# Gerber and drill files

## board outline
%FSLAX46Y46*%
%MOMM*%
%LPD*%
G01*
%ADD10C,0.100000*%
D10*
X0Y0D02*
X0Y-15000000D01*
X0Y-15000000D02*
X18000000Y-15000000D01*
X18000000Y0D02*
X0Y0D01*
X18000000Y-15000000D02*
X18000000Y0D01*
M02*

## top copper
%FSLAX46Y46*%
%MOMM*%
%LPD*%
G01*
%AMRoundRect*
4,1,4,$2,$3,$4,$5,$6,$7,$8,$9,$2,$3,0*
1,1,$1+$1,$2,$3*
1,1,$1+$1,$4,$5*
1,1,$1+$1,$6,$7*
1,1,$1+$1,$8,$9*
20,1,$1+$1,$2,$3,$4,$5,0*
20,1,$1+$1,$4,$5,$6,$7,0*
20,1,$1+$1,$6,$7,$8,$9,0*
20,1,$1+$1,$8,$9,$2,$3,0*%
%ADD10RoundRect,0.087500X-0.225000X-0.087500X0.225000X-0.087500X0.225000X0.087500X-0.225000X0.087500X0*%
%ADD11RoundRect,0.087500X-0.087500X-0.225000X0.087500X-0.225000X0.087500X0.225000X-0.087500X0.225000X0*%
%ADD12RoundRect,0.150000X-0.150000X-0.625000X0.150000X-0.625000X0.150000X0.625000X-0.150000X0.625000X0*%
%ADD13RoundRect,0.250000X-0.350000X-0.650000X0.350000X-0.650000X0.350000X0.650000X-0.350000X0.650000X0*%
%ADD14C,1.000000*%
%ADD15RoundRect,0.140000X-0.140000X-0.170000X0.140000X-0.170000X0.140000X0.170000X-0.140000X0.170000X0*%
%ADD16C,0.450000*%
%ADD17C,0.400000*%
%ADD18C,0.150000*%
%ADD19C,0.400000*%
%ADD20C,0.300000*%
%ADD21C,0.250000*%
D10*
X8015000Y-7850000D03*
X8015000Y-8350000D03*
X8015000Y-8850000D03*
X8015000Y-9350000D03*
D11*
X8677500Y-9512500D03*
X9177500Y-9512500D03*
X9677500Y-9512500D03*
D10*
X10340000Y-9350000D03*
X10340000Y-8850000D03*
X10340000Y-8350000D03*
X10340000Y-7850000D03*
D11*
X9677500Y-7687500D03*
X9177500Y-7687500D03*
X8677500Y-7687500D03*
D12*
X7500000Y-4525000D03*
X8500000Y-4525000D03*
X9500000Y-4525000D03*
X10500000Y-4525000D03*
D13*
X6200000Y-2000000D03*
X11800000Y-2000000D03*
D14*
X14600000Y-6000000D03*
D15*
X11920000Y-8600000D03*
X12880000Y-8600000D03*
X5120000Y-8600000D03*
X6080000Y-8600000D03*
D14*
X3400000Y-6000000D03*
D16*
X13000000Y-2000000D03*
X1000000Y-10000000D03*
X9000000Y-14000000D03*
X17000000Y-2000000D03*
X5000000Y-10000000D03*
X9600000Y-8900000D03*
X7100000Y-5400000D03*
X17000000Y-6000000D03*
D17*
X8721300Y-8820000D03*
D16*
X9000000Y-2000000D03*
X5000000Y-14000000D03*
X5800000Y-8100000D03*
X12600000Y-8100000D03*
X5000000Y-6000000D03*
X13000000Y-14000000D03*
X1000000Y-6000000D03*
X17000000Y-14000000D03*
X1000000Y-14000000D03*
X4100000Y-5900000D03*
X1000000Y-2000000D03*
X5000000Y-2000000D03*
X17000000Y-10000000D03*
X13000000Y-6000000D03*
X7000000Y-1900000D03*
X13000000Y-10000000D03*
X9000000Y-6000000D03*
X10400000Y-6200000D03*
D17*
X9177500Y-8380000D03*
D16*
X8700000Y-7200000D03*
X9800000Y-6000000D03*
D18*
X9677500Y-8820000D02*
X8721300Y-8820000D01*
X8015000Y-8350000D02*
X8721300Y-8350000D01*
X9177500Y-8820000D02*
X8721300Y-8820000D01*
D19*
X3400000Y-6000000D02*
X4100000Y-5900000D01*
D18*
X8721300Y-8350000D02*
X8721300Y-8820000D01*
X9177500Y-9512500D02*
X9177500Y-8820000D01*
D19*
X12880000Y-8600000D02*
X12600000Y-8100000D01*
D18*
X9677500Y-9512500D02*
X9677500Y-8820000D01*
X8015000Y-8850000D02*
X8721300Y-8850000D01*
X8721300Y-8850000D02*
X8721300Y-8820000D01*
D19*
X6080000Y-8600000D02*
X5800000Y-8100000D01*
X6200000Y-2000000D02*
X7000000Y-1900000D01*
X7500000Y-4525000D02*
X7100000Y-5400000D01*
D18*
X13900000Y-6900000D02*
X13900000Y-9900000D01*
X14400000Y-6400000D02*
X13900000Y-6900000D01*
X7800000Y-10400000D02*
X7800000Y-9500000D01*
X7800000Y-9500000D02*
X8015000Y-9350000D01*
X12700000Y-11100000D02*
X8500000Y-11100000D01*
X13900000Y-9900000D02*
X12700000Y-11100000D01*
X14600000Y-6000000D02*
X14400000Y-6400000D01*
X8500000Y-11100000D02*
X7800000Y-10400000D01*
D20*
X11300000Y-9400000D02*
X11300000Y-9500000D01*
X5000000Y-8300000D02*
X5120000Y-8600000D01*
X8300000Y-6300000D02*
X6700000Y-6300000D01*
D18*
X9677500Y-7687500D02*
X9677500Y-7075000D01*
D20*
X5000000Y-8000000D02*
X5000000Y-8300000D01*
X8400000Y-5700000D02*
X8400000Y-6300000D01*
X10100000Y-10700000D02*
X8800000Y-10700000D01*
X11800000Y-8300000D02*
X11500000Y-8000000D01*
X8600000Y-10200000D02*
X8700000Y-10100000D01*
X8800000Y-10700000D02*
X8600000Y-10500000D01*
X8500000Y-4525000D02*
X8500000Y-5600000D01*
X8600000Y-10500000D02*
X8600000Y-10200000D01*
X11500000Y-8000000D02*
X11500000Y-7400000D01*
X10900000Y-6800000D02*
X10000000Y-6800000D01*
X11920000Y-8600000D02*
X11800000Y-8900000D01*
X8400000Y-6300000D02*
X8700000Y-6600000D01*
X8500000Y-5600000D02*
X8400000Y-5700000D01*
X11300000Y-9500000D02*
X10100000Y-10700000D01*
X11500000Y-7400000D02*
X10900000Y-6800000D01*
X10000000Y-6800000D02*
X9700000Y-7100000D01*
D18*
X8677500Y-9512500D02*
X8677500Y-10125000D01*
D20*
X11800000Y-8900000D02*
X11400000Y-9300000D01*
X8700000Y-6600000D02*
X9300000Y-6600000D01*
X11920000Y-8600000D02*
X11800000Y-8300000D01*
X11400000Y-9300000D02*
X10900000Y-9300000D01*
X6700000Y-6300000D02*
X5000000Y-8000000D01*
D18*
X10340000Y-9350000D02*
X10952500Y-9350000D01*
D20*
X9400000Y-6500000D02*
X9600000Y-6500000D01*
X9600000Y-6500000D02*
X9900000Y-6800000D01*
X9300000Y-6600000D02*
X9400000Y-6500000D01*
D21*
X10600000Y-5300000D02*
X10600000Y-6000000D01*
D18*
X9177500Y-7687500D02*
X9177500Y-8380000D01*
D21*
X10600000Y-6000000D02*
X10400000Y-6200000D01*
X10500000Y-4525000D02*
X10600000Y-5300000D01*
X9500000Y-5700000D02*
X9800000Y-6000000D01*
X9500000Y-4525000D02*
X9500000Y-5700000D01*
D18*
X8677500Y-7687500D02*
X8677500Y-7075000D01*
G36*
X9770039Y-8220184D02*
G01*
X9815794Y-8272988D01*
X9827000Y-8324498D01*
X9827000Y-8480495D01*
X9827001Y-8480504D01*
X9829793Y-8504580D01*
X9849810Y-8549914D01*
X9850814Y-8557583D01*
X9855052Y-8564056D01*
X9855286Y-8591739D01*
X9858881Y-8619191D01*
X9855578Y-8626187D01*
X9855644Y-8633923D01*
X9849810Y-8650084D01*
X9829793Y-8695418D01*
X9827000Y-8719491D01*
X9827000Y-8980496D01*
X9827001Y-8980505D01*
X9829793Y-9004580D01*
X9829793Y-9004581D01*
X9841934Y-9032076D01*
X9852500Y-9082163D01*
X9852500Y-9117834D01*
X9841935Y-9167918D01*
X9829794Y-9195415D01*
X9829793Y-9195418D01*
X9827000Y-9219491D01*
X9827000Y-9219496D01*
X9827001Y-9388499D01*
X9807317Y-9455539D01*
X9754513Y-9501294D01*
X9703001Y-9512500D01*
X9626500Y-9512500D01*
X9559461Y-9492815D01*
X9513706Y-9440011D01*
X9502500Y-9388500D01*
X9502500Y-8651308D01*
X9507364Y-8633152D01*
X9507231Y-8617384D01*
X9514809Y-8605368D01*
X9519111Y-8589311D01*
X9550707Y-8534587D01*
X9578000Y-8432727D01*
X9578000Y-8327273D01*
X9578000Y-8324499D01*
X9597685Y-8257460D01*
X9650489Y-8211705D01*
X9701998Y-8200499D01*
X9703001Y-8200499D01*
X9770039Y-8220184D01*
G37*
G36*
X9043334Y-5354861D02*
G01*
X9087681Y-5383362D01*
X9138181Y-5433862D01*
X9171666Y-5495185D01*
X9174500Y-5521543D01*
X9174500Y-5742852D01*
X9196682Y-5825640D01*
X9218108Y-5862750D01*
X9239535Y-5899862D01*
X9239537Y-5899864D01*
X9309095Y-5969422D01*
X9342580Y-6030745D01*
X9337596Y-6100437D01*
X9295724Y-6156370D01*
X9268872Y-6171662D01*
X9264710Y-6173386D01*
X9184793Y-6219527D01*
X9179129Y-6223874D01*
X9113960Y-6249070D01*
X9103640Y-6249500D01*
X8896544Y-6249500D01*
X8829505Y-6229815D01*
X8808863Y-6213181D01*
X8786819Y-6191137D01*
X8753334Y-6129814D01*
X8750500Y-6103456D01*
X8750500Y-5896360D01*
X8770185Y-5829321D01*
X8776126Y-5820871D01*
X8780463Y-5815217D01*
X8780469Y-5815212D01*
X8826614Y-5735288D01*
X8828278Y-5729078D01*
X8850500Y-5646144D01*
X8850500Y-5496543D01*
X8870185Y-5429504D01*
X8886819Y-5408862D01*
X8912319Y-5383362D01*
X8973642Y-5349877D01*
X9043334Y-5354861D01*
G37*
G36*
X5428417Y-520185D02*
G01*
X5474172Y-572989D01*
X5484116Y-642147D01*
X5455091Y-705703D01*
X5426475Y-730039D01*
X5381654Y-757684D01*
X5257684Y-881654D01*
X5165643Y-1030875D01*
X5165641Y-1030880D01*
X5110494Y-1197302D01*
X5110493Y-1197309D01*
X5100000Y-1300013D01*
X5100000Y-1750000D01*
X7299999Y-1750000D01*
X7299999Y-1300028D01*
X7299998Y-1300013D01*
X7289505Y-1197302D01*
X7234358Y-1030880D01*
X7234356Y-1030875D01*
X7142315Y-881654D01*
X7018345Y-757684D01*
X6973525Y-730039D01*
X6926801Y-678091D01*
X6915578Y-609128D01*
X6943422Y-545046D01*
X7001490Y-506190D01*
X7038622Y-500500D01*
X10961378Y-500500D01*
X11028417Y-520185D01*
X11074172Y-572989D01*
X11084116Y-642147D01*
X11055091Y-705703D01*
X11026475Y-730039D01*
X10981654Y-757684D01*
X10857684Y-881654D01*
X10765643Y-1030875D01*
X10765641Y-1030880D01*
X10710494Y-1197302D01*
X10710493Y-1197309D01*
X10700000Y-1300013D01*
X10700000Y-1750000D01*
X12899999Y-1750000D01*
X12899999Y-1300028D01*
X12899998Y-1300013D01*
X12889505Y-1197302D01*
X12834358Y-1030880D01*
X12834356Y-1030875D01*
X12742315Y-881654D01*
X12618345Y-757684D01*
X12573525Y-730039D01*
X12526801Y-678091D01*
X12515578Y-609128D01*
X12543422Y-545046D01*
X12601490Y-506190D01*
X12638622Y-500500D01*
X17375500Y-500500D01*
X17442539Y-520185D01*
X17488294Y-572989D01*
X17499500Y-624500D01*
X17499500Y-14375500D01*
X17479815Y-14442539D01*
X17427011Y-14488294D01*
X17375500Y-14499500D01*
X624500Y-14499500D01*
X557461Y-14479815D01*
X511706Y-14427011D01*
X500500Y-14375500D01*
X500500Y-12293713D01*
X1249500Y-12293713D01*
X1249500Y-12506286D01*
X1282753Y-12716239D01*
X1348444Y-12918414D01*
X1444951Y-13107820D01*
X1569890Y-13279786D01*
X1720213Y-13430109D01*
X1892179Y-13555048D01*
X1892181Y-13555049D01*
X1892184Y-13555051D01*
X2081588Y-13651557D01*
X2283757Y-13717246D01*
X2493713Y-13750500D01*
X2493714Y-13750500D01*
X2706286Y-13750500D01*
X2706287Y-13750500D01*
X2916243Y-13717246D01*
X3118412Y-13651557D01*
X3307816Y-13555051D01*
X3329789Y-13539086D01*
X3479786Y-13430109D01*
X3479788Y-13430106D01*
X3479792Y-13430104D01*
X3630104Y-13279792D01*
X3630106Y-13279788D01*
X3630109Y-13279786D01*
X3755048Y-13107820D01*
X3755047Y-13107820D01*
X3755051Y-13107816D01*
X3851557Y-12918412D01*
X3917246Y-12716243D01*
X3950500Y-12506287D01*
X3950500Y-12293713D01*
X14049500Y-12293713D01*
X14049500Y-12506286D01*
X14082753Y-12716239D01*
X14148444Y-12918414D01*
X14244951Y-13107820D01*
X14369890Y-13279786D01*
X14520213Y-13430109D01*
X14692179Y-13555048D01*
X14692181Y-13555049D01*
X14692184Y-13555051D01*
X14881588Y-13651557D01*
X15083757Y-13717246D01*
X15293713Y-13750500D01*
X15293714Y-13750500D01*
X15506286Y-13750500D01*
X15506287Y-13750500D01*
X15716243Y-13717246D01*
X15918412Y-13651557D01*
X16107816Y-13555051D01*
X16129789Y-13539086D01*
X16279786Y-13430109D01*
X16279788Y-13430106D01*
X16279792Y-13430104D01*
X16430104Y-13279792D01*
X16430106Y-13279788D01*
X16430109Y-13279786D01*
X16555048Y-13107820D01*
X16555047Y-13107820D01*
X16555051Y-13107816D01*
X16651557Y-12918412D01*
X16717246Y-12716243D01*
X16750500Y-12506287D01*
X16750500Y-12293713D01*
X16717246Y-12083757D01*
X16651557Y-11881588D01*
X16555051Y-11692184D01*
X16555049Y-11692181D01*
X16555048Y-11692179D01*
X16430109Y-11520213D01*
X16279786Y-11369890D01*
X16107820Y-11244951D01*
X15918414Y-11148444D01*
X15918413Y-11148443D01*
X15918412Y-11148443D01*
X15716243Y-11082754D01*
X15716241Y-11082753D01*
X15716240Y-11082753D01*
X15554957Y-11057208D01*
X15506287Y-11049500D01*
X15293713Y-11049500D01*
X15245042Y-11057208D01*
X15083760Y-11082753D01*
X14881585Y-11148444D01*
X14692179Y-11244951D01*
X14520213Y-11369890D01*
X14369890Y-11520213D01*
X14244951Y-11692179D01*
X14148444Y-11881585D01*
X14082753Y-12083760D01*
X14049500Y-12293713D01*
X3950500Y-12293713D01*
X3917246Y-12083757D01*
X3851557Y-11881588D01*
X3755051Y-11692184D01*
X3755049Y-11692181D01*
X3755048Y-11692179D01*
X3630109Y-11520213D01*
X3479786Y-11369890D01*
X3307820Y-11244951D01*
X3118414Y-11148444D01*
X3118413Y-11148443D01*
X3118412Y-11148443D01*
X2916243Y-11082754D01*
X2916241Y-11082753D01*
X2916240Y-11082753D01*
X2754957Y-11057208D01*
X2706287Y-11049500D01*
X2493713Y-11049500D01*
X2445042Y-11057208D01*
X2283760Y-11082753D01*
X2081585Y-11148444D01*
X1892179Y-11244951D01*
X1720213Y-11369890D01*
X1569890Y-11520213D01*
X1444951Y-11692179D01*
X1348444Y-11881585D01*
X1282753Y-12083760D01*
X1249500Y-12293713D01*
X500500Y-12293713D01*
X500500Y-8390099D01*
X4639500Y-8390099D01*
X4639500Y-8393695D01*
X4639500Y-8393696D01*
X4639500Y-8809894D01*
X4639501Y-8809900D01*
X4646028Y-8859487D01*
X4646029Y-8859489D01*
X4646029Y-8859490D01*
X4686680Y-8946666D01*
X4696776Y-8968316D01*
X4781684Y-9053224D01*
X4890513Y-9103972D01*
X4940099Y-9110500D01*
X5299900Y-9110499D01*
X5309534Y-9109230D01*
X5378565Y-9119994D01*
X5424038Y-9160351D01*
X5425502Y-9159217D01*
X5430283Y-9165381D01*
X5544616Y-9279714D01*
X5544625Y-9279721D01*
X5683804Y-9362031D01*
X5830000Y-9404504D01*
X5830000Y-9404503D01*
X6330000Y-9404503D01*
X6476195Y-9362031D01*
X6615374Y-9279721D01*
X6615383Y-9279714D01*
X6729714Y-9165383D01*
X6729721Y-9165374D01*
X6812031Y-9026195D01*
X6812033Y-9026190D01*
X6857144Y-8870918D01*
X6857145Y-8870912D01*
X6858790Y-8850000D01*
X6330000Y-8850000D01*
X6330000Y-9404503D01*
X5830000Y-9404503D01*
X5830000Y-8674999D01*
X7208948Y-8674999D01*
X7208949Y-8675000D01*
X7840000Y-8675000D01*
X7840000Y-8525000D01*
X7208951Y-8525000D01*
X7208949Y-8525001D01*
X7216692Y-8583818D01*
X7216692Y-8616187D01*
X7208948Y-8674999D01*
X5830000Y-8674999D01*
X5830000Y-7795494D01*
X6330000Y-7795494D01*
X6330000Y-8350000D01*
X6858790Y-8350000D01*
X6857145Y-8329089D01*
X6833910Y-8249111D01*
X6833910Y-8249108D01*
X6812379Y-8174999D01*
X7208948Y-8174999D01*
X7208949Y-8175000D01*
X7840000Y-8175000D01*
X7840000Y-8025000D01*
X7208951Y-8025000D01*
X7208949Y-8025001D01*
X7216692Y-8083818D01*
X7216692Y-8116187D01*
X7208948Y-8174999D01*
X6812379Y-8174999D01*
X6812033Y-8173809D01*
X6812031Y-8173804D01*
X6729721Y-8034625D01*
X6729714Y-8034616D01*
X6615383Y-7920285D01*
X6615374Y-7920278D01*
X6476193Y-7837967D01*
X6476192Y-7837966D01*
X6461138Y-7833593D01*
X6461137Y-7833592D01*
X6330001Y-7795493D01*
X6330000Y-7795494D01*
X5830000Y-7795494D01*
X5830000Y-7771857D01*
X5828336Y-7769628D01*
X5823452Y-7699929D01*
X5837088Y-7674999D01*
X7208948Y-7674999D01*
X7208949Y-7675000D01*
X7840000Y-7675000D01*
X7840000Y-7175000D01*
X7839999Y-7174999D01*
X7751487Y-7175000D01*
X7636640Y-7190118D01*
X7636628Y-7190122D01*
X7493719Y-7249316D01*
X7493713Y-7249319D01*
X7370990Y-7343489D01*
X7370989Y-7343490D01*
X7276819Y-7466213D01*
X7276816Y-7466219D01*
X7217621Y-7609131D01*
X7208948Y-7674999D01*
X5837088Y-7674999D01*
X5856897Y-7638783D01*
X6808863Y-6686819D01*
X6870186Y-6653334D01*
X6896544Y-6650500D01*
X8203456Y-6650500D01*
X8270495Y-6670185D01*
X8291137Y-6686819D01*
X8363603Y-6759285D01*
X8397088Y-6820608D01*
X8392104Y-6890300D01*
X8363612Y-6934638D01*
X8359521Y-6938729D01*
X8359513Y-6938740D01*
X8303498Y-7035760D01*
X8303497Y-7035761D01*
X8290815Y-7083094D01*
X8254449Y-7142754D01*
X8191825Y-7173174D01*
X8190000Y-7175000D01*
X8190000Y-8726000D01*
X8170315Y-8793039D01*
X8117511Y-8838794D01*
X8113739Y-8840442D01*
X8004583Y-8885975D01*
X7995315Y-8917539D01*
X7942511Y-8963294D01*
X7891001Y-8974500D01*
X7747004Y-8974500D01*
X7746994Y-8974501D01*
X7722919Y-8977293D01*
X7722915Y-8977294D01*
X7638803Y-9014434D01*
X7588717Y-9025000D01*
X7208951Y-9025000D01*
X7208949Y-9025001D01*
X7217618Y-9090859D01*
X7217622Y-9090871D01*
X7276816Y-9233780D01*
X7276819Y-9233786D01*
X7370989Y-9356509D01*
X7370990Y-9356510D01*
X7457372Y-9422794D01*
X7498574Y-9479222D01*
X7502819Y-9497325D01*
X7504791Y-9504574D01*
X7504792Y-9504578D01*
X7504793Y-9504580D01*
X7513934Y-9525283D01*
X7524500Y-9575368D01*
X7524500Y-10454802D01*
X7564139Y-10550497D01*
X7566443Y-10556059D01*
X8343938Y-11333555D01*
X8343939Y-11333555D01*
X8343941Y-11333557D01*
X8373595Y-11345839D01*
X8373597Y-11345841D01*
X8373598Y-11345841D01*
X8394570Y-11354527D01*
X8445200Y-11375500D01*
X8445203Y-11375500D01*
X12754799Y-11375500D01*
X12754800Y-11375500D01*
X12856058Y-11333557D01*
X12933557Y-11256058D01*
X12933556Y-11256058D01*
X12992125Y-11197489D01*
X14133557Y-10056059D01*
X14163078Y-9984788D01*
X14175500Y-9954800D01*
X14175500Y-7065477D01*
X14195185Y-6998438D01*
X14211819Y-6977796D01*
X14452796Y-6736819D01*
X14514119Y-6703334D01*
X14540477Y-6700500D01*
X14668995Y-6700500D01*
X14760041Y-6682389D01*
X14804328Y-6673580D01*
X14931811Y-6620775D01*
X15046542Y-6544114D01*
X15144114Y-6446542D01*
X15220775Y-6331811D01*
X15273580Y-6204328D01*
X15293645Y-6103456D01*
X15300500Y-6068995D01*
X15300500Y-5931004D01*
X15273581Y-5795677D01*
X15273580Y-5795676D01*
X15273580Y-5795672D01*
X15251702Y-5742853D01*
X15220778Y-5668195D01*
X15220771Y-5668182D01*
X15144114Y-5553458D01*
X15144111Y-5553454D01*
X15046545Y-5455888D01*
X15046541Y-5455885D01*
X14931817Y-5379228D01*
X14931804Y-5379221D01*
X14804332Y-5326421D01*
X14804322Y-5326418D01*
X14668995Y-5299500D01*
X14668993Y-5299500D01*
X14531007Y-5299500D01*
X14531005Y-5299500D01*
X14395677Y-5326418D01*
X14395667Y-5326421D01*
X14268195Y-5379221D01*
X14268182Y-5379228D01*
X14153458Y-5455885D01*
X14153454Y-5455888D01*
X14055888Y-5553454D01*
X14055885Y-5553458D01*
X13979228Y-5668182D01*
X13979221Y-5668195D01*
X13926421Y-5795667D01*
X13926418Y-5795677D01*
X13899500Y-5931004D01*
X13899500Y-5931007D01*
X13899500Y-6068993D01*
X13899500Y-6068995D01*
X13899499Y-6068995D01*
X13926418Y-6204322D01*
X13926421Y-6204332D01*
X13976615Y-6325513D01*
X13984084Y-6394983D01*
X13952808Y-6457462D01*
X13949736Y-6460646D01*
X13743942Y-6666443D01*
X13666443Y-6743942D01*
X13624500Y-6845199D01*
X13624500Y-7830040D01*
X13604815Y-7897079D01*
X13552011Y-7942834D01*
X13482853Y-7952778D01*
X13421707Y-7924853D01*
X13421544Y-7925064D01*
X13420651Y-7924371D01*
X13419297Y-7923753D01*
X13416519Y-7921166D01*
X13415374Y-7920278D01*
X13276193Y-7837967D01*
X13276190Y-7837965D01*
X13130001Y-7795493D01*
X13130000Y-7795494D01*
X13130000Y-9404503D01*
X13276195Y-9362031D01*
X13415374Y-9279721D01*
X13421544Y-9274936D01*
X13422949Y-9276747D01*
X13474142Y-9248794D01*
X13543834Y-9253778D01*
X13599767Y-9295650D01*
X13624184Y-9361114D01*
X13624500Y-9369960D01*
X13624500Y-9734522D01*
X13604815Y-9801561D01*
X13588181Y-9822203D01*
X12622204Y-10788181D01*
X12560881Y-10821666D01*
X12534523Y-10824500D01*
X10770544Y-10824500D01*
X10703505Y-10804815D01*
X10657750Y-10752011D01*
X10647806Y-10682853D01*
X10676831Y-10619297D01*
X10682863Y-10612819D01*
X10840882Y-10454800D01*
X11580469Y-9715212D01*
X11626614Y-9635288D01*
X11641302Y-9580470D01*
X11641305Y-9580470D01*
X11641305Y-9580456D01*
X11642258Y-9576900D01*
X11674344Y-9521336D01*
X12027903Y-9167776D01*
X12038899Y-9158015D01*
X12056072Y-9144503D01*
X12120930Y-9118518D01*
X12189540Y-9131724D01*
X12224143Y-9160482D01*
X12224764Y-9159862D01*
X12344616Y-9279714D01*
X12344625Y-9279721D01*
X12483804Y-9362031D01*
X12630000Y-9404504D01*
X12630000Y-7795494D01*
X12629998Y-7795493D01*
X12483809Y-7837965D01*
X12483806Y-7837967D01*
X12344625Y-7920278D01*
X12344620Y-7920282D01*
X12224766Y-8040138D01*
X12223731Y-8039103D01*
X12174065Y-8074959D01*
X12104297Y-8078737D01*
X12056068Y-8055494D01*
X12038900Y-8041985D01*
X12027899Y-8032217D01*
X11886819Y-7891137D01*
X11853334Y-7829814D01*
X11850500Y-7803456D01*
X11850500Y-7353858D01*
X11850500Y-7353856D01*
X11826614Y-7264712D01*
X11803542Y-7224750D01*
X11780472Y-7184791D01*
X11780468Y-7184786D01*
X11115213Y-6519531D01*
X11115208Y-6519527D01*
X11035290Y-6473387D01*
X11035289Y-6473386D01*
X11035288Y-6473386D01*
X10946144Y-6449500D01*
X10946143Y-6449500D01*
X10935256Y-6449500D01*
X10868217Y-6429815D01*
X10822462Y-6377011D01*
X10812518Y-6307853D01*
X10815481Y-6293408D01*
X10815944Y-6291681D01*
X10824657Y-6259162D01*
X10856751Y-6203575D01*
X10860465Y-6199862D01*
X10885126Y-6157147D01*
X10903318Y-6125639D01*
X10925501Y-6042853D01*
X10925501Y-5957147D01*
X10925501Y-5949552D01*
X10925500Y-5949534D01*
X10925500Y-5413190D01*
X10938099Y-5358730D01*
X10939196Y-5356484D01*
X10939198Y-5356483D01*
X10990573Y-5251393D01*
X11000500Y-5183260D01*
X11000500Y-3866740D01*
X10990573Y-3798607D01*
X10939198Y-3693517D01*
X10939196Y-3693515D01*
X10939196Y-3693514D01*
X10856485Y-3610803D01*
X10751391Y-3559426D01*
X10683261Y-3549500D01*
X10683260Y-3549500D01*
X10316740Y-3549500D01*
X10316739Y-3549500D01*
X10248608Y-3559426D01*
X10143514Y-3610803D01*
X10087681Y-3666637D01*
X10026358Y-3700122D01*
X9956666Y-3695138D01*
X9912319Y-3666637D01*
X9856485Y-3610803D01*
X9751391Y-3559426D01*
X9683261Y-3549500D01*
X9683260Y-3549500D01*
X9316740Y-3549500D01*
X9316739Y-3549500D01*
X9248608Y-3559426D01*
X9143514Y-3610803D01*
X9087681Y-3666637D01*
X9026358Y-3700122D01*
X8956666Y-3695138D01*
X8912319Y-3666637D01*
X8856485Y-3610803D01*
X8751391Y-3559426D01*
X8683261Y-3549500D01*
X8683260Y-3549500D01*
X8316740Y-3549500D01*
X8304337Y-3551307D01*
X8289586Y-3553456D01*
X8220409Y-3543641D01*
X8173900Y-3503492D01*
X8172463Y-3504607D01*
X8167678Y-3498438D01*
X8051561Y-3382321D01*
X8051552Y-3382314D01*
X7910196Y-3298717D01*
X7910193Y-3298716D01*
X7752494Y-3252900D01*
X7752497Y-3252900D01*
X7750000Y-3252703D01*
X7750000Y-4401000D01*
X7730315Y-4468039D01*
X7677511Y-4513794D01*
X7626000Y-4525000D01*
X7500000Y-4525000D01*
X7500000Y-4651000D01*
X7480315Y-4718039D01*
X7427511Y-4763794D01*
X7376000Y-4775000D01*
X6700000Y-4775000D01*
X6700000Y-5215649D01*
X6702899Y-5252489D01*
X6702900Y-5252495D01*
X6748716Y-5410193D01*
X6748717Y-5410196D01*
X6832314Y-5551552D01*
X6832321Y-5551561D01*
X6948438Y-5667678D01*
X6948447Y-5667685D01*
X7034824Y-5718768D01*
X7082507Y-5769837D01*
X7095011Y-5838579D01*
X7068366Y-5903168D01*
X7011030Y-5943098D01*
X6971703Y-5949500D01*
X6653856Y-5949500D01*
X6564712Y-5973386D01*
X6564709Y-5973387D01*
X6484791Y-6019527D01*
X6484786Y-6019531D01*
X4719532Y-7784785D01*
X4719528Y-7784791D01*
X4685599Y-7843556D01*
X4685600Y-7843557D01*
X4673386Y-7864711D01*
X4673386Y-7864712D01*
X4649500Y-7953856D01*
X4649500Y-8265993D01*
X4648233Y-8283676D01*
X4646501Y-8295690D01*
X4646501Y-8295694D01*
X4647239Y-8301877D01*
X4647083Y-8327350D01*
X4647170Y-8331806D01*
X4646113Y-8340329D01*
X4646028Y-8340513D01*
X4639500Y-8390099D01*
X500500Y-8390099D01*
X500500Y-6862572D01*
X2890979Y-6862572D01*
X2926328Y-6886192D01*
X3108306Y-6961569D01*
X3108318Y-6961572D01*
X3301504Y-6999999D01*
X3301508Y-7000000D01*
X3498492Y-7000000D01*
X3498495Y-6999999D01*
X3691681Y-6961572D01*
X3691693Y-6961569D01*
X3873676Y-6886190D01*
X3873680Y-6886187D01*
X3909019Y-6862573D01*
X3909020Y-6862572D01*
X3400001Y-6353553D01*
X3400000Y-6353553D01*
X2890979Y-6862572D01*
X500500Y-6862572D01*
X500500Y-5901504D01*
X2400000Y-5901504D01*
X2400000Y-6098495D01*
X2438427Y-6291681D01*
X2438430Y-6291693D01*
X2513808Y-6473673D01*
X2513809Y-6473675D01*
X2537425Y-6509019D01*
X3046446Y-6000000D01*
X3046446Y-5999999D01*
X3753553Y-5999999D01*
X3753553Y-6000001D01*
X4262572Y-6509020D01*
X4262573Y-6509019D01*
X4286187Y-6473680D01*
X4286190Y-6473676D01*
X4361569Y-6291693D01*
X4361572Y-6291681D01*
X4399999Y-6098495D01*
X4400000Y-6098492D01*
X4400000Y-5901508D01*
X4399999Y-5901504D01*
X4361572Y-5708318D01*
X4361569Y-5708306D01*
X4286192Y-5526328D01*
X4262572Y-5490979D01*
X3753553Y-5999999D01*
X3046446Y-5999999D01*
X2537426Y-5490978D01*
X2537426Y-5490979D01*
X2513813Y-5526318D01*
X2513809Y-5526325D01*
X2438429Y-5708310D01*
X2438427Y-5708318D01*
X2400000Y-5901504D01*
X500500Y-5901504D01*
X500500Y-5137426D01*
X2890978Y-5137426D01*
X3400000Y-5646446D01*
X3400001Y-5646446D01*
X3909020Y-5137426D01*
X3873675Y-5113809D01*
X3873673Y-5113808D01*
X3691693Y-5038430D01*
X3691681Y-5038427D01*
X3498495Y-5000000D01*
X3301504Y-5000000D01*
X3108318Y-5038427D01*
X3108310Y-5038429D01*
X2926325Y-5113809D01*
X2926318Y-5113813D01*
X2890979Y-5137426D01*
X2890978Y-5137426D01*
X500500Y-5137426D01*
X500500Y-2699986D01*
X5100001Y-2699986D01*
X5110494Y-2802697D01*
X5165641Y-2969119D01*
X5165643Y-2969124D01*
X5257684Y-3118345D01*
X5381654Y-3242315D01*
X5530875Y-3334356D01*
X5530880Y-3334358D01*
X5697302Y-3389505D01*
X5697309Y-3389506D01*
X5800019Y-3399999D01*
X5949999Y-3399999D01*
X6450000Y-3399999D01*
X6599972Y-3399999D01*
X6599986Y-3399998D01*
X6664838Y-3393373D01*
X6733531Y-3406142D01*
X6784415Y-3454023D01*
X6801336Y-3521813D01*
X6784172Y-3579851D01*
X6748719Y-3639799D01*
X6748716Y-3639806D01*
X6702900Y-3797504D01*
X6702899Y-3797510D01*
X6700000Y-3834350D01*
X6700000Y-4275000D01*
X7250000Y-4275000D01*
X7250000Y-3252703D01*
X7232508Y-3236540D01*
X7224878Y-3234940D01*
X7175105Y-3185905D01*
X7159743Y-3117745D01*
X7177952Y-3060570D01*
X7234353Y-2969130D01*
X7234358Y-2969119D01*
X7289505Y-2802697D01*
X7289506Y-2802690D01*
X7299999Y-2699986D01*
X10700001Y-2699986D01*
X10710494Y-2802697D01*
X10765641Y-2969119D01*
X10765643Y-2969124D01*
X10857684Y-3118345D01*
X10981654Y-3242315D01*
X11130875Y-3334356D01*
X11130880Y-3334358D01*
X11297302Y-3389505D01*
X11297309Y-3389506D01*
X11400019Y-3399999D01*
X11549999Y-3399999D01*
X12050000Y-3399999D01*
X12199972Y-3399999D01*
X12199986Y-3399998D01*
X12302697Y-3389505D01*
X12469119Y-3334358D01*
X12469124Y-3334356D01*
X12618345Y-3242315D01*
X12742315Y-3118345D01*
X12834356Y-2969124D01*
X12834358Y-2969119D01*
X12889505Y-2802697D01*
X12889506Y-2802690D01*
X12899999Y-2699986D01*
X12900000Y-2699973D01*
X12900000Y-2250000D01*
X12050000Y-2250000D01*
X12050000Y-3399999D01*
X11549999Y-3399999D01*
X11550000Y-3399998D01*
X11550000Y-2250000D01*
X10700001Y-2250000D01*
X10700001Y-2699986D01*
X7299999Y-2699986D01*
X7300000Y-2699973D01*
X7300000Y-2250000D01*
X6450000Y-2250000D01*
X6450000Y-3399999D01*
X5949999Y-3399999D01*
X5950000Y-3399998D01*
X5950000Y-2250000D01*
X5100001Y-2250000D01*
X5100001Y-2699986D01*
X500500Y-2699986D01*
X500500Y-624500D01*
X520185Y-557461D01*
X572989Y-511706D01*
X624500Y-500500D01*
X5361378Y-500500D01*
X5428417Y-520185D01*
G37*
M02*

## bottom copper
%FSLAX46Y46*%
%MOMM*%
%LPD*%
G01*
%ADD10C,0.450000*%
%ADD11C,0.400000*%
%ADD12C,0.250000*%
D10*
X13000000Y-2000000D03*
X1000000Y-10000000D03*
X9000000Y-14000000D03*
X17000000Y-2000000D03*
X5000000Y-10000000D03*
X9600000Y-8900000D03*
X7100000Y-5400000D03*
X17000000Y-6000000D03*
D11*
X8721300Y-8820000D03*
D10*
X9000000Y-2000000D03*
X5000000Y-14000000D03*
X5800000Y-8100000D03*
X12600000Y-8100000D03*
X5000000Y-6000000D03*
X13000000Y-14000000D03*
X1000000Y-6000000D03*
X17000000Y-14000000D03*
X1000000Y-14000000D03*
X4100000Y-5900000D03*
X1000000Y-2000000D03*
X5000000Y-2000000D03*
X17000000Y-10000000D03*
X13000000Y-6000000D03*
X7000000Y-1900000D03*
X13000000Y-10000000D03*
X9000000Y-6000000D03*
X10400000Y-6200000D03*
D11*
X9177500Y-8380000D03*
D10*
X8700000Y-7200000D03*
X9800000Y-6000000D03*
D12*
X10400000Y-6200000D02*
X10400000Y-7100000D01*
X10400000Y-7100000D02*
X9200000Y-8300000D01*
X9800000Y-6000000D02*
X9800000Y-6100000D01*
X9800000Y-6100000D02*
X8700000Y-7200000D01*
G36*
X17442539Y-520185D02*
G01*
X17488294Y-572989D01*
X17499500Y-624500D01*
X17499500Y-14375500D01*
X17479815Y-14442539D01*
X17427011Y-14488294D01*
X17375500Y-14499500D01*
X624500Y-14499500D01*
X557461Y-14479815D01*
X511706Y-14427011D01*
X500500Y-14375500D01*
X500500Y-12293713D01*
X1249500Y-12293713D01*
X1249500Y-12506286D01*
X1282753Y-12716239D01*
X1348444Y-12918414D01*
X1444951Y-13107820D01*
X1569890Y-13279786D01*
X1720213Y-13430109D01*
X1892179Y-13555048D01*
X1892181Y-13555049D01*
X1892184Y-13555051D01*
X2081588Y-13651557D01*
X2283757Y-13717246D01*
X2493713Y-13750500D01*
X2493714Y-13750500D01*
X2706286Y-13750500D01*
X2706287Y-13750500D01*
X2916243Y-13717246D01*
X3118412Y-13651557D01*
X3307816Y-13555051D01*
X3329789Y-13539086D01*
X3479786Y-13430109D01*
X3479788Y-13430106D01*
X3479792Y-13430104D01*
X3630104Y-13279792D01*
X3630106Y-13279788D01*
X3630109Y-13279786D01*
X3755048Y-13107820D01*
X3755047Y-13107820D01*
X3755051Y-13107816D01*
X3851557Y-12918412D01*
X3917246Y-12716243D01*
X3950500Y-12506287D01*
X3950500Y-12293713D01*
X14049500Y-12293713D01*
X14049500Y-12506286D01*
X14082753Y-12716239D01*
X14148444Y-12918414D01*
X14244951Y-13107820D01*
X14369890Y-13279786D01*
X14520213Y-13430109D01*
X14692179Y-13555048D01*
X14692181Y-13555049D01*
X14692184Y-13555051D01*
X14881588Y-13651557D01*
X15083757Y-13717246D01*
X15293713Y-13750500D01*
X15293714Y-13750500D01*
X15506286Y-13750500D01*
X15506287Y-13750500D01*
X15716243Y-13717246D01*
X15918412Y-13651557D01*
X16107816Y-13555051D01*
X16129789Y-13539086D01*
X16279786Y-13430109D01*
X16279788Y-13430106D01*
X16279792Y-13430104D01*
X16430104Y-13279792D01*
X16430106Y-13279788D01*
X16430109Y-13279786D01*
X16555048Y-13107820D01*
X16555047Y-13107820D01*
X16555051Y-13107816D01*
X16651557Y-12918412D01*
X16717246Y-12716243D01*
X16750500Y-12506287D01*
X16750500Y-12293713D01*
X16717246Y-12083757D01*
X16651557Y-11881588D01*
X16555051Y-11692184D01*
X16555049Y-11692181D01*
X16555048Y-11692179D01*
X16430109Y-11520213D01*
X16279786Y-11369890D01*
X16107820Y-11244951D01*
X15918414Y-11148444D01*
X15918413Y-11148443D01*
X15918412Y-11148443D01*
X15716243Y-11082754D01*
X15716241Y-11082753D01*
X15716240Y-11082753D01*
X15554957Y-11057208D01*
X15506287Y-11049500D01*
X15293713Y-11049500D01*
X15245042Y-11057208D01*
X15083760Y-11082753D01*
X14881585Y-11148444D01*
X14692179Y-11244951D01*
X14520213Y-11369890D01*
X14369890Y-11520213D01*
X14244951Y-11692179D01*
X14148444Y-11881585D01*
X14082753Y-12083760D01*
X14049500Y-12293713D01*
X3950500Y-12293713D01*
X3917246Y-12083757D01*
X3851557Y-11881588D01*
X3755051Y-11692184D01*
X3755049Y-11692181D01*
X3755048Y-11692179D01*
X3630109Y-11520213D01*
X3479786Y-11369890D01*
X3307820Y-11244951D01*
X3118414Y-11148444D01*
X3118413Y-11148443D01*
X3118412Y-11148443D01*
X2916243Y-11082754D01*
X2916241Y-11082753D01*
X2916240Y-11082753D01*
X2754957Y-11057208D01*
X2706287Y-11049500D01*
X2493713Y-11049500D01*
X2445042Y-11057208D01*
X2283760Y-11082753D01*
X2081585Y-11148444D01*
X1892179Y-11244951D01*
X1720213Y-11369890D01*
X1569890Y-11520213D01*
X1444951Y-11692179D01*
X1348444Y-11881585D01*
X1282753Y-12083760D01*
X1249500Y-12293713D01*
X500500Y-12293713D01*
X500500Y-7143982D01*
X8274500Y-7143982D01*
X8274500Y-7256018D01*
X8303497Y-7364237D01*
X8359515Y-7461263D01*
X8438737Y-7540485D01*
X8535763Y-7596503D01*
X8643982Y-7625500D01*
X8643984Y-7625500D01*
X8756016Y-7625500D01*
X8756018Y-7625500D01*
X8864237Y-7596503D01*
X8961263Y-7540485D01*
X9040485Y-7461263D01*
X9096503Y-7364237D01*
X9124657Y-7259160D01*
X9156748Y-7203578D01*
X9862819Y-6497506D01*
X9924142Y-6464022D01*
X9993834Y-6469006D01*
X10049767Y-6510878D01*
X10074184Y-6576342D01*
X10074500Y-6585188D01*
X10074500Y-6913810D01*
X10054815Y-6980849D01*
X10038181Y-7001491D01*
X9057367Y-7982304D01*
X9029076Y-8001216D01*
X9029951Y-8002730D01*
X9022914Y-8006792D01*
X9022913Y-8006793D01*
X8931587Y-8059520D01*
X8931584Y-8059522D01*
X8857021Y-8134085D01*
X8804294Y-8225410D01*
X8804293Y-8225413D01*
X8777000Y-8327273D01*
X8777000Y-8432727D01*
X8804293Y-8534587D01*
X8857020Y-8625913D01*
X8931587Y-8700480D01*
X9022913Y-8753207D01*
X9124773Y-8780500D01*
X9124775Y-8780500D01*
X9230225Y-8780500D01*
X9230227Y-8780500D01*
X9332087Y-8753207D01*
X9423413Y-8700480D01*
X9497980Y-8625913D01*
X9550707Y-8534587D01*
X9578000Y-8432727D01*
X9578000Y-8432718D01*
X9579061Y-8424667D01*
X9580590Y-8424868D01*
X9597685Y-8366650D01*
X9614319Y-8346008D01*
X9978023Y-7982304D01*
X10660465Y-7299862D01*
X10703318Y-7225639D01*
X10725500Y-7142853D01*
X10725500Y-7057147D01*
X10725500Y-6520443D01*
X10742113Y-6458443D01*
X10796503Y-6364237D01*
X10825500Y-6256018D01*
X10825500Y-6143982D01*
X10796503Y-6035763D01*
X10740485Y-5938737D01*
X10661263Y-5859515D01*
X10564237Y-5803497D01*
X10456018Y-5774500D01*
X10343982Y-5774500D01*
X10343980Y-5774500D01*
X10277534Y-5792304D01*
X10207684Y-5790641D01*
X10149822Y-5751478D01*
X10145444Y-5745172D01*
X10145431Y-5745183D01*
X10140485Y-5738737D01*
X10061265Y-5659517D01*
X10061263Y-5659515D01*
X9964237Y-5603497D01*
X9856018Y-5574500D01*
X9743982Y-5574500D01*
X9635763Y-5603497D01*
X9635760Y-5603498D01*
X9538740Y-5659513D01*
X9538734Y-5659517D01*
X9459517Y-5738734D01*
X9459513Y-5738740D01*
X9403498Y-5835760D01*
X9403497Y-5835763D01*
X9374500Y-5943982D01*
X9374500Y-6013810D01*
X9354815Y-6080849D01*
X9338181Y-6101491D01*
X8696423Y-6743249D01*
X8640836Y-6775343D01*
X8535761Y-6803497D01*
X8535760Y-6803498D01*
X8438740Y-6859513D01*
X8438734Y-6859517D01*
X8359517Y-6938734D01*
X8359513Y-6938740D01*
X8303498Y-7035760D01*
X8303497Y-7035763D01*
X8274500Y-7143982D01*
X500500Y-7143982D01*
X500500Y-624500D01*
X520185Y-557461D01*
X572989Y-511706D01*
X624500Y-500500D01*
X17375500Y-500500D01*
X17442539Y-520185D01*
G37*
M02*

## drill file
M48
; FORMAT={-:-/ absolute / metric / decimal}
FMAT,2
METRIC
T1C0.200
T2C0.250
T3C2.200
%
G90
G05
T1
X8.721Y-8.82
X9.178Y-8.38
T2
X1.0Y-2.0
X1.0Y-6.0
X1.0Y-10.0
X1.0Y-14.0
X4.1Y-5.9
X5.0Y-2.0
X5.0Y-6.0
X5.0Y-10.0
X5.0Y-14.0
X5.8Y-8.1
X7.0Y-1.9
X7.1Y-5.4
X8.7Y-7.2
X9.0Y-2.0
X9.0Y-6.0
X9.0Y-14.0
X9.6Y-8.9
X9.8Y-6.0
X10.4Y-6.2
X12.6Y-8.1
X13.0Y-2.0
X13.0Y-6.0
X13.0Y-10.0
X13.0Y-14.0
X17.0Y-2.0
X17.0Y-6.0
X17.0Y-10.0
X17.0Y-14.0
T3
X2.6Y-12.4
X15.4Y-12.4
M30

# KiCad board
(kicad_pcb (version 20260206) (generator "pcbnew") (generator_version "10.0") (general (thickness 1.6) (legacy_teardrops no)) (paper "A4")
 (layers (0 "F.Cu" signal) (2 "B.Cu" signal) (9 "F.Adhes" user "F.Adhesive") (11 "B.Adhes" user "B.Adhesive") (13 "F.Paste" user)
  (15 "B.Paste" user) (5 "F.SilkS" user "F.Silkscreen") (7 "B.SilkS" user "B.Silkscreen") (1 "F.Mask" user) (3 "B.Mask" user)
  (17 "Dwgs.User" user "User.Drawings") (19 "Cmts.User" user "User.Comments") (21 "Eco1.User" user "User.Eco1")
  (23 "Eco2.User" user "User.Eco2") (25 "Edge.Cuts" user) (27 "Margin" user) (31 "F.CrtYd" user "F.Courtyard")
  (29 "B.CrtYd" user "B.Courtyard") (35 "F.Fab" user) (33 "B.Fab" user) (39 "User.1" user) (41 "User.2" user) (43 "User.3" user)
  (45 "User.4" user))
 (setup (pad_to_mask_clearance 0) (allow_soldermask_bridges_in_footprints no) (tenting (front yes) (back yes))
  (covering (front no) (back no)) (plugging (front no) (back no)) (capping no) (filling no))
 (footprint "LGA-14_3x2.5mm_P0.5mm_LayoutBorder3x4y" (layer "F.Cu") (at 9.1775 8.6)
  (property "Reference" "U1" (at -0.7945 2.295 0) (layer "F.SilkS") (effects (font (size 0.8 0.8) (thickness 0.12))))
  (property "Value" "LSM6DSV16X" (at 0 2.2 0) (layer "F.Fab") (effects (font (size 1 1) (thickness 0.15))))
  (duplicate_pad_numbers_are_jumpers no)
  (pad "1" smd roundrect (at -1.1625 -0.75) (size 0.625 0.35) (layers "F.Cu" "F.Mask" "F.Paste") (roundrect_rratio 0.25) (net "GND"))
  (pad "2" smd roundrect (at -1.1625 -0.25) (size 0.625 0.35) (layers "F.Cu" "F.Mask" "F.Paste") (roundrect_rratio 0.25) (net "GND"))
  (pad "3" smd roundrect (at -1.1625 0.25) (size 0.625 0.35) (layers "F.Cu" "F.Mask" "F.Paste") (roundrect_rratio 0.25) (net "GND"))
  (pad "4" smd roundrect (at -1.1625 0.75) (size 0.625 0.35) (layers "F.Cu" "F.Mask" "F.Paste") (roundrect_rratio 0.25) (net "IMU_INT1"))
  (pad "5" smd roundrect (at -0.5 0.9125) (size 0.35 0.625) (layers "F.Cu" "F.Mask" "F.Paste") (roundrect_rratio 0.25) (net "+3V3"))
  (pad "6" smd roundrect (at 0 0.9125) (size 0.35 0.625) (layers "F.Cu" "F.Mask" "F.Paste") (roundrect_rratio 0.25) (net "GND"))
  (pad "7" smd roundrect (at 0.5 0.9125) (size 0.35 0.625) (layers "F.Cu" "F.Mask" "F.Paste") (roundrect_rratio 0.25) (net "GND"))
  (pad "8" smd roundrect (at 1.1625 0.75) (size 0.625 0.35) (layers "F.Cu" "F.Mask" "F.Paste") (roundrect_rratio 0.25) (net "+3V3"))
  (pad "9" smd roundrect (at 1.1625 0.25) (size 0.625 0.35) (layers "F.Cu" "F.Mask" "F.Paste") (roundrect_rratio 0.25))
  (pad "10" smd roundrect (at 1.1625 -0.25) (size 0.625 0.35) (layers "F.Cu" "F.Mask" "F.Paste") (roundrect_rratio 0.25))
  (pad "11" smd roundrect (at 1.1625 -0.75) (size 0.625 0.35) (layers "F.Cu" "F.Mask" "F.Paste") (roundrect_rratio 0.25))
  (pad "12" smd roundrect (at 0.5 -0.9125) (size 0.35 0.625) (layers "F.Cu" "F.Mask" "F.Paste") (roundrect_rratio 0.25) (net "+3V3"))
  (pad "13" smd roundrect (at 0 -0.9125) (size 0.35 0.625) (layers "F.Cu" "F.Mask" "F.Paste") (roundrect_rratio 0.25) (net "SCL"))
  (pad "14" smd roundrect (at -0.5 -0.9125) (size 0.35 0.625) (layers "F.Cu" "F.Mask" "F.Paste") (roundrect_rratio 0.25) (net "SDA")))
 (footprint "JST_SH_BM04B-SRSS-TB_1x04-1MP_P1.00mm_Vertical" (layer "F.Cu") (at 9 3.2)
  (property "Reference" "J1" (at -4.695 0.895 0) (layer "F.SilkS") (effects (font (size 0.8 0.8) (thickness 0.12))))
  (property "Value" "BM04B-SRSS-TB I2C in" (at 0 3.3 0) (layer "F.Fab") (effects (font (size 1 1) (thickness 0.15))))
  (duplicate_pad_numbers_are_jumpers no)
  (pad "1" smd roundrect (at -1.5 1.325) (size 0.6 1.55) (layers "F.Cu" "F.Mask" "F.Paste") (roundrect_rratio 0.25) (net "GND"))
  (pad "2" smd roundrect (at -0.5 1.325) (size 0.6 1.55) (layers "F.Cu" "F.Mask" "F.Paste") (roundrect_rratio 0.25) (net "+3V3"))
  (pad "3" smd roundrect (at 0.5 1.325) (size 0.6 1.55) (layers "F.Cu" "F.Mask" "F.Paste") (roundrect_rratio 0.25) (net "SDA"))
  (pad "4" smd roundrect (at 1.5 1.325) (size 0.6 1.55) (layers "F.Cu" "F.Mask" "F.Paste") (roundrect_rratio 0.25) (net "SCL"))
  (pad "MP" smd roundrect (at -2.8 -1.2) (size 1.2 1.8) (layers "F.Cu" "F.Mask" "F.Paste") (roundrect_rratio 0.208333) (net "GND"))
  (pad "MP" smd roundrect (at 2.8 -1.2) (size 1.2 1.8) (layers "F.Cu" "F.Mask" "F.Paste") (roundrect_rratio 0.208333) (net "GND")))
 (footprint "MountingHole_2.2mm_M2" (layer "F.Cu") (at 15.4 12.4)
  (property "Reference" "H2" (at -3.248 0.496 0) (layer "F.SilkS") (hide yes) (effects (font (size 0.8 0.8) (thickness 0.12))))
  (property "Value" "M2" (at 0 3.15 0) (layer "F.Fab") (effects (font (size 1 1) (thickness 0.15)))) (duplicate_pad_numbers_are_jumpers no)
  (pad "" np_thru_hole circle (at 0 0) (size 2.2 2.2) (drill 2.2) (layers "*.Cu" "*.Mask")))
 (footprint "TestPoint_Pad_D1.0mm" (layer "F.Cu") (at 14.6 6)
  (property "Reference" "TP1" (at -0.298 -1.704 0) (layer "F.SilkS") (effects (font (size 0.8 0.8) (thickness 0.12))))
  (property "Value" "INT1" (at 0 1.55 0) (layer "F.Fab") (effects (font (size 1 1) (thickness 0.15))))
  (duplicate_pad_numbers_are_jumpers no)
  (pad "1" smd circle (at 0 0) (size 1 1) (layers "F.Cu" "F.Mask") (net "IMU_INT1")))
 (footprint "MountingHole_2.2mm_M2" (layer "F.Cu") (at 2.6 12.4)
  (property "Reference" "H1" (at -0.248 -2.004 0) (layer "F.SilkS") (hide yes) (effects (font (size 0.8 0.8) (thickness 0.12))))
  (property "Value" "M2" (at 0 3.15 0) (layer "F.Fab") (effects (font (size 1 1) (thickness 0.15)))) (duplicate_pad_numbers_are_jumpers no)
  (pad "" np_thru_hole circle (at 0 0) (size 2.2 2.2) (drill 2.2) (layers "*.Cu" "*.Mask")))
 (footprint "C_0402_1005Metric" (layer "F.Cu") (at 12.4 8.6)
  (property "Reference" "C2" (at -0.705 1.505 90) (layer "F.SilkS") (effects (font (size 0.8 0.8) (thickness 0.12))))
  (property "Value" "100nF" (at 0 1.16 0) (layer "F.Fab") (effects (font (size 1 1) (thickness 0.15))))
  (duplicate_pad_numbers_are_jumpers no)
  (pad "1" smd roundrect (at -0.48 0) (size 0.56 0.62) (layers "F.Cu" "F.Mask" "F.Paste") (roundrect_rratio 0.25) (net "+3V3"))
  (pad "2" smd roundrect (at 0.48 0) (size 0.56 0.62) (layers "F.Cu" "F.Mask" "F.Paste") (roundrect_rratio 0.25) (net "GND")))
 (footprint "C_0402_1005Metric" (layer "F.Cu") (at 5.6 8.6)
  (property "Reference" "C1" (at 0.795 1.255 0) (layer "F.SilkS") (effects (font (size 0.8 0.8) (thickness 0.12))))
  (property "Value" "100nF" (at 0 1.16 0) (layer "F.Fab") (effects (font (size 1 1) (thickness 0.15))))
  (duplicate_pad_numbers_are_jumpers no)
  (pad "1" smd roundrect (at -0.48 0) (size 0.56 0.62) (layers "F.Cu" "F.Mask" "F.Paste") (roundrect_rratio 0.25) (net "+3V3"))
  (pad "2" smd roundrect (at 0.48 0) (size 0.56 0.62) (layers "F.Cu" "F.Mask" "F.Paste") (roundrect_rratio 0.25) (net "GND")))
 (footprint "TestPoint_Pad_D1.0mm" (layer "F.Cu") (at 3.4 6)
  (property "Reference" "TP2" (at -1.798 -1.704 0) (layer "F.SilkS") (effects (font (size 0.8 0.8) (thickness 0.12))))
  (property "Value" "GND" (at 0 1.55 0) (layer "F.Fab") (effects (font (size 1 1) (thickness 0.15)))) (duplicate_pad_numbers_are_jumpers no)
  (pad "1" smd circle (at 0 0) (size 1 1) (layers "F.Cu" "F.Mask") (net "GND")))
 (gr_line (start 0 0) (end 0 15) (stroke (width 0.1) (type default)) (layer "Edge.Cuts"))
 (gr_line (start 0 15) (end 18 15) (stroke (width 0.1) (type default)) (layer "Edge.Cuts"))
 (gr_line (start 18 0) (end 0 0) (stroke (width 0.1) (type default)) (layer "Edge.Cuts"))
 (gr_line (start 18 15) (end 18 0) (stroke (width 0.1) (type default)) (layer "Edge.Cuts"))
 (segment (start 9.6775 8.82) (end 8.7213 8.82) (width 0.15) (layer "F.Cu") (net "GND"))
 (segment (start 8.015 8.35) (end 8.7213 8.35) (width 0.15) (layer "F.Cu") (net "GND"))
 (segment (start 9.1775 8.82) (end 8.7213 8.82) (width 0.15) (layer "F.Cu") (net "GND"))
 (segment (start 3.4 6) (end 4.1 5.9) (width 0.4) (layer "F.Cu") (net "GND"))
 (segment (start 8.7213 8.35) (end 8.7213 8.82) (width 0.15) (layer "F.Cu") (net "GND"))
 (segment (start 9.1775 9.5125) (end 9.1775 8.82) (width 0.15) (layer "F.Cu") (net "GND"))
 (segment (start 12.88 8.6) (end 12.6 8.1) (width 0.4) (layer "F.Cu") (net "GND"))
 (segment (start 9.6775 9.5125) (end 9.6775 8.82) (width 0.15) (layer "F.Cu") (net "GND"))
 (segment (start 8.015 8.85) (end 8.7213 8.85) (width 0.15) (layer "F.Cu") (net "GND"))
 (segment (start 8.7213 8.85) (end 8.7213 8.82) (width 0.15) (layer "F.Cu") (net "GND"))
 (segment (start 6.08 8.6) (end 5.8 8.1) (width 0.4) (layer "F.Cu") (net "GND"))
 (segment (start 6.2 2) (end 7 1.9) (width 0.4) (layer "F.Cu") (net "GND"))
 (segment (start 7.5 4.525) (end 7.1 5.4) (width 0.4) (layer "F.Cu") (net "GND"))
 (via (at 13 2) (size 0.45) (drill 0.25) (layers "F.Cu" "B.Cu") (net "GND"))
 (via (at 1 10) (size 0.45) (drill 0.25) (layers "F.Cu" "B.Cu") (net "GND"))
 (via (at 9 14) (size 0.45) (drill 0.25) (layers "F.Cu" "B.Cu") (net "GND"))
 (via (at 17 2) (size 0.45) (drill 0.25) (layers "F.Cu" "B.Cu") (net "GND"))
 (via (at 5 10) (size 0.45) (drill 0.25) (layers "F.Cu" "B.Cu") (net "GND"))
 (via (at 9.6 8.9) (size 0.45) (drill 0.25) (layers "F.Cu" "B.Cu") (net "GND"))
 (via (at 7.1 5.4) (size 0.45) (drill 0.25) (layers "F.Cu" "B.Cu") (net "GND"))
 (via (at 17 6) (size 0.45) (drill 0.25) (layers "F.Cu" "B.Cu") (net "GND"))
 (via (at 8.7213 8.82) (size 0.4) (drill 0.2) (layers "F.Cu" "B.Cu") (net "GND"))
 (via (at 9 2) (size 0.45) (drill 0.25) (layers "F.Cu" "B.Cu") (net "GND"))
 (via (at 5 14) (size 0.45) (drill 0.25) (layers "F.Cu" "B.Cu") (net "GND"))
 (via (at 5.8 8.1) (size 0.45) (drill 0.25) (layers "F.Cu" "B.Cu") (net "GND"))
 (via (at 12.6 8.1) (size 0.45) (drill 0.25) (layers "F.Cu" "B.Cu") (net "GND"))
 (via (at 5 6) (size 0.45) (drill 0.25) (layers "F.Cu" "B.Cu") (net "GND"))
 (via (at 13 14) (size 0.45) (drill 0.25) (layers "F.Cu" "B.Cu") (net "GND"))
 (via (at 1 6) (size 0.45) (drill 0.25) (layers "F.Cu" "B.Cu") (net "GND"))
 (via (at 17 14) (size 0.45) (drill 0.25) (layers "F.Cu" "B.Cu") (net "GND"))
 (via (at 1 14) (size 0.45) (drill 0.25) (layers "F.Cu" "B.Cu") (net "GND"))
 (via (at 4.1 5.9) (size 0.45) (drill 0.25) (layers "F.Cu" "B.Cu") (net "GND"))
 (via (at 1 2) (size 0.45) (drill 0.25) (layers "F.Cu" "B.Cu") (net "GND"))
 (via (at 5 2) (size 0.45) (drill 0.25) (layers "F.Cu" "B.Cu") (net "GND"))
 (via (at 17 10) (size 0.45) (drill 0.25) (layers "F.Cu" "B.Cu") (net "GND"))
 (via (at 13 6) (size 0.45) (drill 0.25) (layers "F.Cu" "B.Cu") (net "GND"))
 (via (at 7 1.9) (size 0.45) (drill 0.25) (layers "F.Cu" "B.Cu") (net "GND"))
 (via (at 13 10) (size 0.45) (drill 0.25) (layers "F.Cu" "B.Cu") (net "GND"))
 (via (at 9 6) (size 0.45) (drill 0.25) (layers "F.Cu" "B.Cu") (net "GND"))
 (segment (start 13.9 6.9) (end 13.9 9.9) (width 0.15) (layer "F.Cu") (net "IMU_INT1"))
 (segment (start 14.4 6.4) (end 13.9 6.9) (width 0.15) (layer "F.Cu") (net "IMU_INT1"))
 (segment (start 7.8 10.4) (end 7.8 9.5) (width 0.15) (layer "F.Cu") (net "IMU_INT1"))
 (segment (start 7.8 9.5) (end 8.015 9.35) (width 0.15) (layer "F.Cu") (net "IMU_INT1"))
 (segment (start 12.7 11.1) (end 8.5 11.1) (width 0.15) (layer "F.Cu") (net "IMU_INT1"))
 (segment (start 13.9 9.9) (end 12.7 11.1) (width 0.15) (layer "F.Cu") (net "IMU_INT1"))
 (segment (start 14.6 6) (end 14.4 6.4) (width 0.15) (layer "F.Cu") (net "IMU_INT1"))
 (segment (start 8.5 11.1) (end 7.8 10.4) (width 0.15) (layer "F.Cu") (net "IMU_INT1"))
 (segment (start 11.3 9.4) (end 11.3 9.5) (width 0.3) (layer "F.Cu") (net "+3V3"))
 (segment (start 5 8.3) (end 5.12 8.6) (width 0.3) (layer "F.Cu") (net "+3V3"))
 (segment (start 8.3 6.3) (end 6.7 6.3) (width 0.3) (layer "F.Cu") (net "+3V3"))
 (segment (start 9.6775 7.6875) (end 9.6775 7.075) (width 0.15) (layer "F.Cu") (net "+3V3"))
 (segment (start 5 8) (end 5 8.3) (width 0.3) (layer "F.Cu") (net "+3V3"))
 (segment (start 8.4 5.7) (end 8.4 6.3) (width 0.3) (layer "F.Cu") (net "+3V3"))
 (segment (start 10.1 10.7) (end 8.8 10.7) (width 0.3) (layer "F.Cu") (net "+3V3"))
 (segment (start 11.8 8.3) (end 11.5 8) (width 0.3) (layer "F.Cu") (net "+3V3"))
 (segment (start 8.6 10.2) (end 8.7 10.1) (width 0.3) (layer "F.Cu") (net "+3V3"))
 (segment (start 8.8 10.7) (end 8.6 10.5) (width 0.3) (layer "F.Cu") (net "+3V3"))
 (segment (start 8.5 4.525) (end 8.5 5.6) (width 0.3) (layer "F.Cu") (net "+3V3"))
 (segment (start 8.6 10.5) (end 8.6 10.2) (width 0.3) (layer "F.Cu") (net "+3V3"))
 (segment (start 11.5 8) (end 11.5 7.4) (width 0.3) (layer "F.Cu") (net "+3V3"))
 (segment (start 10.9 6.8) (end 10 6.8) (width 0.3) (layer "F.Cu") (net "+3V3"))
 (segment (start 11.92 8.6) (end 11.8 8.9) (width 0.3) (layer "F.Cu") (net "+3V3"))
 (segment (start 8.4 6.3) (end 8.7 6.6) (width 0.3) (layer "F.Cu") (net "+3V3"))
 (segment (start 8.5 5.6) (end 8.4 5.7) (width 0.3) (layer "F.Cu") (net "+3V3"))
 (segment (start 11.3 9.5) (end 10.1 10.7) (width 0.3) (layer "F.Cu") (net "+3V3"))
 (segment (start 11.5 7.4) (end 10.9 6.8) (width 0.3) (layer "F.Cu") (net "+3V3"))
 (segment (start 10 6.8) (end 9.7 7.1) (width 0.3) (layer "F.Cu") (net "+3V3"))
 (segment (start 8.6775 9.5125) (end 8.6775 10.125) (width 0.15) (layer "F.Cu") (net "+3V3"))
 (segment (start 11.8 8.9) (end 11.4 9.3) (width 0.3) (layer "F.Cu") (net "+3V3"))
 (segment (start 8.7 6.6) (end 9.3 6.6) (width 0.3) (layer "F.Cu") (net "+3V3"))
 (segment (start 11.92 8.6) (end 11.8 8.3) (width 0.3) (layer "F.Cu") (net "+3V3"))
 (segment (start 11.4 9.3) (end 10.9 9.3) (width 0.3) (layer "F.Cu") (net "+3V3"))
 (segment (start 6.7 6.3) (end 5 8) (width 0.3) (layer "F.Cu") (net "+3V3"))
 (segment (start 10.34 9.35) (end 10.9525 9.35) (width 0.15) (layer "F.Cu") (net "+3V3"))
 (segment (start 9.4 6.5) (end 9.6 6.5) (width 0.3) (layer "F.Cu") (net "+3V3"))
 (segment (start 9.6 6.5) (end 9.9 6.8) (width 0.3) (layer "F.Cu") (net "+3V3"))
 (segment (start 9.3 6.6) (end 9.4 6.5) (width 0.3) (layer "F.Cu") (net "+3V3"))
 (segment (start 10.6 5.3) (end 10.6 6) (width 0.25) (layer "F.Cu") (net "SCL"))
 (segment (start 9.1775 7.6875) (end 9.1775 8.38) (width 0.15) (layer "F.Cu") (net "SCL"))
 (segment (start 10.6 6) (end 10.4 6.2) (width 0.25) (layer "F.Cu") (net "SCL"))
 (segment (start 10.5 4.525) (end 10.6 5.3) (width 0.25) (layer "F.Cu") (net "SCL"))
 (via (at 10.4 6.2) (size 0.45) (drill 0.25) (layers "F.Cu" "B.Cu") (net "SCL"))
 (via (at 9.1775 8.38) (size 0.4) (drill 0.2) (layers "F.Cu" "B.Cu") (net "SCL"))
 (segment (start 10.4 6.2) (end 10.4 7.1) (width 0.25) (layer "B.Cu") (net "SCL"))
 (segment (start 10.4 7.1) (end 9.2 8.3) (width 0.25) (layer "B.Cu") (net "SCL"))
 (segment (start 9.5 5.7) (end 9.8 6) (width 0.25) (layer "F.Cu") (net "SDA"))
 (segment (start 9.5 4.525) (end 9.5 5.7) (width 0.25) (layer "F.Cu") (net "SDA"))
 (segment (start 8.6775 7.6875) (end 8.6775 7.075) (width 0.15) (layer "F.Cu") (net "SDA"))
 (via (at 8.7 7.2) (size 0.45) (drill 0.25) (layers "F.Cu" "B.Cu") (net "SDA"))
 (via (at 9.8 6) (size 0.45) (drill 0.25) (layers "F.Cu" "B.Cu") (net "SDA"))
 (segment (start 9.8 6) (end 9.8 6.1) (width 0.25) (layer "B.Cu") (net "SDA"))
 (segment (start 9.8 6.1) (end 8.7 7.2) (width 0.25) (layer "B.Cu") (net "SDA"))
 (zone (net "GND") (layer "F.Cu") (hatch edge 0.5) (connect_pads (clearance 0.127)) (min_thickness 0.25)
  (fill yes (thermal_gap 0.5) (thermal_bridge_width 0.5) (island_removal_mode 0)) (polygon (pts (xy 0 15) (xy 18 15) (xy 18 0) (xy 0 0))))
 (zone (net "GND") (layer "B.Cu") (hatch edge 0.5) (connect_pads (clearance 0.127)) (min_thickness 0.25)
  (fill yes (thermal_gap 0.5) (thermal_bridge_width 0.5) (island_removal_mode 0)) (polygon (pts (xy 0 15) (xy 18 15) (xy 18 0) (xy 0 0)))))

